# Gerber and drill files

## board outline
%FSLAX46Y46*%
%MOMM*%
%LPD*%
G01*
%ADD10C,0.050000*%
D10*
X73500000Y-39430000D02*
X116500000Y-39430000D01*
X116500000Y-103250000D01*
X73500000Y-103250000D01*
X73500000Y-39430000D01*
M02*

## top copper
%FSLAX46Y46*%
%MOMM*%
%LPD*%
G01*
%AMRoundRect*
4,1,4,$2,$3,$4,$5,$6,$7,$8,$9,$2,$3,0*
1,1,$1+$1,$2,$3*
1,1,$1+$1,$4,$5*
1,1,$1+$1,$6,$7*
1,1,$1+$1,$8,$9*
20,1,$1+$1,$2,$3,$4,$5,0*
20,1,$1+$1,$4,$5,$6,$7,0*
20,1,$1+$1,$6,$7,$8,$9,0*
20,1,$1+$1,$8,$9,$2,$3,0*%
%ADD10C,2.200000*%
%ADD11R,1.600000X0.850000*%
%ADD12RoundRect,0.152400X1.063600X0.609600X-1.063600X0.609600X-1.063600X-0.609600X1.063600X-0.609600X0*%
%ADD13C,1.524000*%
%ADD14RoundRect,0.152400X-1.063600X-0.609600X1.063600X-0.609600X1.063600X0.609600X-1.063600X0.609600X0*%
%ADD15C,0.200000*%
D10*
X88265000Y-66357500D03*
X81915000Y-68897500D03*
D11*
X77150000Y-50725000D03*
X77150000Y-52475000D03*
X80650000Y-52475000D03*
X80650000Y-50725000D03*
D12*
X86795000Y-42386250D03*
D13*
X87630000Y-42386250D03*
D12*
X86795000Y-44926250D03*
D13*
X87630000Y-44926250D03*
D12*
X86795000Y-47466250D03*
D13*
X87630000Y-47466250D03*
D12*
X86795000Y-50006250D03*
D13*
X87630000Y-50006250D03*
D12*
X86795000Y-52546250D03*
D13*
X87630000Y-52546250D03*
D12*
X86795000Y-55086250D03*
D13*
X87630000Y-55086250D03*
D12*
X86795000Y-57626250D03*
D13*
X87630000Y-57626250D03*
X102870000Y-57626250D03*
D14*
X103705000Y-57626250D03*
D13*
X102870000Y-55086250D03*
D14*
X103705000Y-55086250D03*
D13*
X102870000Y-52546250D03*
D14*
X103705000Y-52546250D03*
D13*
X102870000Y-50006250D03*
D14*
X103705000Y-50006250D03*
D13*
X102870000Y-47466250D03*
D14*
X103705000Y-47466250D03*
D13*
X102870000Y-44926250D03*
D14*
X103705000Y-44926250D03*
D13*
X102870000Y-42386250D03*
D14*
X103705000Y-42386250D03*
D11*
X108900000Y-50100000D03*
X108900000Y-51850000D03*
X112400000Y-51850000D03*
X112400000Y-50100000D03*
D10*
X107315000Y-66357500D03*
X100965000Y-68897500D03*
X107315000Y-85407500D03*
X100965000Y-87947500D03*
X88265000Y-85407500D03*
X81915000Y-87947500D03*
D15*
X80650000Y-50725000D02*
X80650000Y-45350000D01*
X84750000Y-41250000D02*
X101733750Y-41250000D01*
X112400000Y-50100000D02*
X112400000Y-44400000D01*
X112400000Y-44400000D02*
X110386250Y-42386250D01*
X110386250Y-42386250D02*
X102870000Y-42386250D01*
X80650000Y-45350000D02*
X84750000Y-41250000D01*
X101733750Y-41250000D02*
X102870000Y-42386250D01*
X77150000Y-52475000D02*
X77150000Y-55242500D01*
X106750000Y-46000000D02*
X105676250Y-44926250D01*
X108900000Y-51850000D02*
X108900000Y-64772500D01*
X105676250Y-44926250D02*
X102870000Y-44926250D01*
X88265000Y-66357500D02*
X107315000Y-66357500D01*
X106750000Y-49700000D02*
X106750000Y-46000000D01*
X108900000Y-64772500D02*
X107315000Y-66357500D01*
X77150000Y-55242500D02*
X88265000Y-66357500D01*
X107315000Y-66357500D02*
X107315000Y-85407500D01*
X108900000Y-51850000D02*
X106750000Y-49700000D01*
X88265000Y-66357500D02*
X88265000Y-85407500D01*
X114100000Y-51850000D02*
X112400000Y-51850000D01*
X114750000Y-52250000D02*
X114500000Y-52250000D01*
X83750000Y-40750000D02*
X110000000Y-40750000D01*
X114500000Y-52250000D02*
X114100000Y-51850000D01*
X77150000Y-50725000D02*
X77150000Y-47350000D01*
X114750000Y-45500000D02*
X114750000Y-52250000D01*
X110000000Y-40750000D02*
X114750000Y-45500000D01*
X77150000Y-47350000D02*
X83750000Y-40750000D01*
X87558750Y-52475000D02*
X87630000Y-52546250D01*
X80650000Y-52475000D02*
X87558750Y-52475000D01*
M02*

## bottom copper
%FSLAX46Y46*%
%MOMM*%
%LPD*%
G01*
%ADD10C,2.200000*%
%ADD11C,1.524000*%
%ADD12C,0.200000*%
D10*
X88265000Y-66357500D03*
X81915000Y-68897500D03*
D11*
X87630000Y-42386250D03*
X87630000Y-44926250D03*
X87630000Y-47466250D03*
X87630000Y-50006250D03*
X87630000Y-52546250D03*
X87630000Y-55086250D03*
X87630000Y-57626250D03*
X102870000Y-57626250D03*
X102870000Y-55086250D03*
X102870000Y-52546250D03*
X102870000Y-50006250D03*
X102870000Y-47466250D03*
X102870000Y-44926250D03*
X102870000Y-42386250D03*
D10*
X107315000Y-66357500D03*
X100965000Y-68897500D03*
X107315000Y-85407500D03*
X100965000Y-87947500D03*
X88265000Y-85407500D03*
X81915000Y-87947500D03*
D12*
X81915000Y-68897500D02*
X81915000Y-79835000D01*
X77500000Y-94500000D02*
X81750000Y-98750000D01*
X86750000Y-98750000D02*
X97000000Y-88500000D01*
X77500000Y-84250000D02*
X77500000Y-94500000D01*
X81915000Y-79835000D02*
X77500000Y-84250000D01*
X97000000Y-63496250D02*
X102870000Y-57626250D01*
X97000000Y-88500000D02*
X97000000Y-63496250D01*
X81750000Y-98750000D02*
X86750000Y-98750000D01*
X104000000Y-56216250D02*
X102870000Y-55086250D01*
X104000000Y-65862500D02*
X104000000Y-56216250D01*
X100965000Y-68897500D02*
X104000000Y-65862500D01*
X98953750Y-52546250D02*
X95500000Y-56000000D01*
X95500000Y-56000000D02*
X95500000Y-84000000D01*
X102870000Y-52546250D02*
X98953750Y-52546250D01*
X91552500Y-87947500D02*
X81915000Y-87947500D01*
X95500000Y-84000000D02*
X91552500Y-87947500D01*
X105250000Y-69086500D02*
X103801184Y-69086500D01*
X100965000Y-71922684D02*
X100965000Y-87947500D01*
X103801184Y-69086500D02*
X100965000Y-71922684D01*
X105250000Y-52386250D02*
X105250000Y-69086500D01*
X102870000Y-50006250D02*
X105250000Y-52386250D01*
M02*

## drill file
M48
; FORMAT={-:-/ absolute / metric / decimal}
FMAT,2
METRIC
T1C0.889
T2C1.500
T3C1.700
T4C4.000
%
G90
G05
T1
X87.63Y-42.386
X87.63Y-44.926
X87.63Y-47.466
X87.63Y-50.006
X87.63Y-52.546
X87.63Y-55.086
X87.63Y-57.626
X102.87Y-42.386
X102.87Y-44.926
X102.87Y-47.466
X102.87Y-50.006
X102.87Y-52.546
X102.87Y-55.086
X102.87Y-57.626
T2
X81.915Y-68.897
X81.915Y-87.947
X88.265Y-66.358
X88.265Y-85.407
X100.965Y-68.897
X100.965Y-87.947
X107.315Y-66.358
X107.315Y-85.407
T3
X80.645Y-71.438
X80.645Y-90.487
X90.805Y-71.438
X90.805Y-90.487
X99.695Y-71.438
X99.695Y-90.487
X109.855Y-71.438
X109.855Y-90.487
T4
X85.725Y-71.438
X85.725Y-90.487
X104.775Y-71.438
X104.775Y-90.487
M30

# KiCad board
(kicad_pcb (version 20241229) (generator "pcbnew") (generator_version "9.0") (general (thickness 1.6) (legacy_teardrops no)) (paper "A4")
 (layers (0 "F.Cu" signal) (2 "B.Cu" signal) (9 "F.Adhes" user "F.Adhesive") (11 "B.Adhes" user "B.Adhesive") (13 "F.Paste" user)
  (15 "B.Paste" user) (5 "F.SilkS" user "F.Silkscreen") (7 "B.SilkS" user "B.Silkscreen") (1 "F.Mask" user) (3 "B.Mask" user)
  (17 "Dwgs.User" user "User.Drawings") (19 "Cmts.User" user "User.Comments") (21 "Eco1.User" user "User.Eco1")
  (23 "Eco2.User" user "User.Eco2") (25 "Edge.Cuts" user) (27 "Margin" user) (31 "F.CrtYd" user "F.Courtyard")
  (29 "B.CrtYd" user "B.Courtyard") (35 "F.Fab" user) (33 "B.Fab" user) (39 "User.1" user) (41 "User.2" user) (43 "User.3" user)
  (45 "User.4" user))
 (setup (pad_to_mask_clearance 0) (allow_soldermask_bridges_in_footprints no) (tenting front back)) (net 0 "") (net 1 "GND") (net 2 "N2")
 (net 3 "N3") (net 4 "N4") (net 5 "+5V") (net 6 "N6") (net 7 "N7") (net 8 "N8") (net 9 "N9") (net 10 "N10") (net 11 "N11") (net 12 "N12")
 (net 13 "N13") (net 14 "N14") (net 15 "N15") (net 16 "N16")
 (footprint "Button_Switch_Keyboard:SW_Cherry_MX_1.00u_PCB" (layer "F.Cu") (at 88.265 66.3575)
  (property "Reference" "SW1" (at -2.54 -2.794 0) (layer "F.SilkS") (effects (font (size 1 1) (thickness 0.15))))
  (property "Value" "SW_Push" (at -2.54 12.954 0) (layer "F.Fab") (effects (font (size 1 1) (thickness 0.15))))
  (pad "" np_thru_hole circle (at -7.62 5.08) (size 1.7 1.7) (drill 1.7) (layers "*.Cu" "*.Mask"))
  (pad "" np_thru_hole circle (at -2.54 5.08) (size 4 4) (drill 4) (layers "*.Cu" "*.Mask"))
  (pad "" np_thru_hole circle (at 2.54 5.08) (size 1.7 1.7) (drill 1.7) (layers "*.Cu" "*.Mask"))
  (pad "1" thru_hole circle (at 0 0) (size 2.2 2.2) (drill 1.5) (layers "*.Cu" "*.Mask") (remove_unused_layers no) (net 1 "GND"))
  (pad "2" thru_hole circle (at -6.35 2.54) (size 2.2 2.2) (drill 1.5) (layers "*.Cu" "*.Mask") (remove_unused_layers no) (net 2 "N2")))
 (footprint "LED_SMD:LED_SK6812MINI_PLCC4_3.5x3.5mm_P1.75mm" (layer "F.Cu") (at 78.9 51.6)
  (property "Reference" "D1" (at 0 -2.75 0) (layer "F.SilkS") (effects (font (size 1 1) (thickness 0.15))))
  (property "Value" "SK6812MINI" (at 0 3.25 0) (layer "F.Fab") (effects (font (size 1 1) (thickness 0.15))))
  (pad "1" smd rect (at -1.75 -0.875) (size 1.6 0.85) (layers "F.Cu" "F.Mask" "F.Paste") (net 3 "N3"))
  (pad "2" smd rect (at -1.75 0.875) (size 1.6 0.85) (layers "F.Cu" "F.Mask" "F.Paste") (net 1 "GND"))
  (pad "3" smd rect (at 1.75 0.875) (size 1.6 0.85) (layers "F.Cu" "F.Mask" "F.Paste") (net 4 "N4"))
  (pad "4" smd rect (at 1.75 -0.875) (size 1.6 0.85) (layers "F.Cu" "F.Mask" "F.Paste") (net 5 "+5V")))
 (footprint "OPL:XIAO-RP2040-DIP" (layer "F.Cu") (at 95.25 50.00625)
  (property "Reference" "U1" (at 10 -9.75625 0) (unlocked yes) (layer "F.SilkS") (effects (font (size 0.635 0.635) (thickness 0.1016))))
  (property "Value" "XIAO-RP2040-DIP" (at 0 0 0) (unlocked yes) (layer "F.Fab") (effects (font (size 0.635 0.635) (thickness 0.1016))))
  (pad "1" smd roundrect (at -8.455 -7.62 180) (size 2.432 1.524) (layers "F.Cu" "F.Mask") (roundrect_rratio 0.1) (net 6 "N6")
   (thermal_bridge_angle 45))
  (pad "1" thru_hole circle (at -7.62 -7.62 180) (size 1.524 1.524) (drill 0.889) (layers "*.Cu" "*.Mask") (remove_unused_layers no)
   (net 6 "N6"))
  (pad "2" smd roundrect (at -8.455 -5.08 180) (size 2.432 1.524) (layers "F.Cu" "F.Mask") (roundrect_rratio 0.1) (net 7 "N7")
   (thermal_bridge_angle 45))
  (pad "2" thru_hole circle (at -7.62 -5.08 180) (size 1.524 1.524) (drill 0.889) (layers "*.Cu" "*.Mask") (remove_unused_layers no)
   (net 7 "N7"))
  (pad "3" smd roundrect (at -8.455 -2.54 180) (size 2.432 1.524) (layers "F.Cu" "F.Mask") (roundrect_rratio 0.1) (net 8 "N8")
   (thermal_bridge_angle 45))
  (pad "3" thru_hole circle (at -7.62 -2.54 180) (size 1.524 1.524) (drill 0.889) (layers "*.Cu" "*.Mask") (remove_unused_layers no)
   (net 8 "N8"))
  (pad "4" smd roundrect (at -8.455 0 180) (size 2.432 1.524) (layers "F.Cu" "F.Mask") (roundrect_rratio 0.1) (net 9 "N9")
   (thermal_bridge_angle 45))
  (pad "4" thru_hole circle (at -7.62 0 180) (size 1.524 1.524) (drill 0.889) (layers "*.Cu" "*.Mask") (remove_unused_layers no)
   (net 9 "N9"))
  (pad "5" smd roundrect (at -8.455 2.54 180) (size 2.432 1.524) (layers "F.Cu" "F.Mask") (roundrect_rratio 0.1) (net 4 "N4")
   (thermal_bridge_angle 45))
  (pad "5" thru_hole circle (at -7.62 2.54 180) (size 1.524 1.524) (drill 0.889) (layers "*.Cu" "*.Mask") (remove_unused_layers no)
   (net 4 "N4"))
  (pad "6" smd roundrect (at -8.455 5.08 180) (size 2.432 1.524) (layers "F.Cu" "F.Mask") (roundrect_rratio 0.1) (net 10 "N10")
   (thermal_bridge_angle 45))
  (pad "6" thru_hole circle (at -7.62 5.08 180) (size 1.524 1.524) (drill 0.889) (layers "*.Cu" "*.Mask") (remove_unused_layers no)
   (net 10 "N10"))
  (pad "7" smd roundrect (at -8.455 7.62 180) (size 2.432 1.524) (layers "F.Cu" "F.Mask") (roundrect_rratio 0.1) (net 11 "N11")
   (thermal_bridge_angle 45))
  (pad "7" thru_hole circle (at -7.62 7.62 180) (size 1.524 1.524) (drill 0.889) (layers "*.Cu" "*.Mask") (remove_unused_layers no)
   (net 11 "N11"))
  (pad "8" thru_hole circle (at 7.62 7.62) (size 1.524 1.524) (drill 0.889) (layers "*.Cu" "*.Mask") (remove_unused_layers no) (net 2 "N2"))
  (pad "8" smd roundrect (at 8.455 7.62) (size 2.432 1.524) (layers "F.Cu" "F.Mask") (roundrect_rratio 0.1) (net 2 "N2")
   (thermal_bridge_angle 45))
  (pad "9" thru_hole circle (at 7.62 5.08) (size 1.524 1.524) (drill 0.889) (layers "*.Cu" "*.Mask") (remove_unused_layers no)
   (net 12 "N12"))
  (pad "9" smd roundrect (at 8.455 5.08) (size 2.432 1.524) (layers "F.Cu" "F.Mask") (roundrect_rratio 0.1) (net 12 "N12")
   (thermal_bridge_angle 45))
  (pad "10" thru_hole circle (at 7.62 2.54) (size 1.524 1.524) (drill 0.889) (layers "*.Cu" "*.Mask") (remove_unused_layers no)
   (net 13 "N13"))
  (pad "10" smd roundrect (at 8.455 2.54) (size 2.432 1.524) (layers "F.Cu" "F.Mask") (roundrect_rratio 0.1) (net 13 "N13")
   (thermal_bridge_angle 45))
  (pad "11" thru_hole circle (at 7.62 0) (size 1.524 1.524) (drill 0.889) (layers "*.Cu" "*.Mask") (remove_unused_layers no) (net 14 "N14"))
  (pad "11" smd roundrect (at 8.455 0) (size 2.432 1.524) (layers "F.Cu" "F.Mask") (roundrect_rratio 0.1) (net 14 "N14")
   (thermal_bridge_angle 45))
  (pad "12" thru_hole circle (at 7.62 -2.54) (size 1.524 1.524) (drill 0.889) (layers "*.Cu" "*.Mask") (remove_unused_layers no)
   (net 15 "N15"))
  (pad "12" smd roundrect (at 8.455 -2.54) (size 2.432 1.524) (layers "F.Cu" "F.Mask") (roundrect_rratio 0.1) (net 15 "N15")
   (thermal_bridge_angle 45))
  (pad "13" thru_hole circle (at 7.62 -5.08) (size 1.524 1.524) (drill 0.889) (layers "*.Cu" "*.Mask") (remove_unused_layers no)
   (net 1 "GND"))
  (pad "13" smd roundrect (at 8.455 -5.08) (size 2.432 1.524) (layers "F.Cu" "F.Mask") (roundrect_rratio 0.1) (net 1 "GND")
   (thermal_bridge_angle 45))
  (pad "14" thru_hole circle (at 7.62 -7.62) (size 1.524 1.524) (drill 0.889) (layers "*.Cu" "*.Mask") (remove_unused_layers no)
   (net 5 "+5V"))
  (pad "14" smd roundrect (at 8.455 -7.62) (size 2.432 1.524) (layers "F.Cu" "F.Mask") (roundrect_rratio 0.1) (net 5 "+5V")
   (thermal_bridge_angle 45)))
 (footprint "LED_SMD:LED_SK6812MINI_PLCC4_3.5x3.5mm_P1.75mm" (layer "F.Cu") (at 110.65 50.975)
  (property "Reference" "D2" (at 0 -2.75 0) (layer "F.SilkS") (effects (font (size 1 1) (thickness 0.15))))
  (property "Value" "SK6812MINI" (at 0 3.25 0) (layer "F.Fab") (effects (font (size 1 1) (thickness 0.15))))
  (pad "1" smd rect (at -1.75 -0.875) (size 1.6 0.85) (layers "F.Cu" "F.Mask" "F.Paste") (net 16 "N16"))
  (pad "2" smd rect (at -1.75 0.875) (size 1.6 0.85) (layers "F.Cu" "F.Mask" "F.Paste") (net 1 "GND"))
  (pad "3" smd rect (at 1.75 0.875) (size 1.6 0.85) (layers "F.Cu" "F.Mask" "F.Paste") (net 3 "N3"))
  (pad "4" smd rect (at 1.75 -0.875) (size 1.6 0.85) (layers "F.Cu" "F.Mask" "F.Paste") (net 5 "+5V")))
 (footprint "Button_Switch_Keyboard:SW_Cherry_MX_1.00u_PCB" (layer "F.Cu") (at 107.315 66.3575)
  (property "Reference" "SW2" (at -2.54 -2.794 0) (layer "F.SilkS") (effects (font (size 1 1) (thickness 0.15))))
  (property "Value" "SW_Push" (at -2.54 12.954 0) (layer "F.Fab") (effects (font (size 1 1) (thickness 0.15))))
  (pad "" np_thru_hole circle (at -7.62 5.08) (size 1.7 1.7) (drill 1.7) (layers "*.Cu" "*.Mask"))
  (pad "" np_thru_hole circle (at -2.54 5.08) (size 4 4) (drill 4) (layers "*.Cu" "*.Mask"))
  (pad "" np_thru_hole circle (at 2.54 5.08) (size 1.7 1.7) (drill 1.7) (layers "*.Cu" "*.Mask"))
  (pad "1" thru_hole circle (at 0 0) (size 2.2 2.2) (drill 1.5) (layers "*.Cu" "*.Mask") (remove_unused_layers no) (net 1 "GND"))
  (pad "2" thru_hole circle (at -6.35 2.54) (size 2.2 2.2) (drill 1.5) (layers "*.Cu" "*.Mask") (remove_unused_layers no) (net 12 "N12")))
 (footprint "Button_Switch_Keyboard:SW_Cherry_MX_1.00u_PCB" (layer "F.Cu") (at 107.315 85.4075)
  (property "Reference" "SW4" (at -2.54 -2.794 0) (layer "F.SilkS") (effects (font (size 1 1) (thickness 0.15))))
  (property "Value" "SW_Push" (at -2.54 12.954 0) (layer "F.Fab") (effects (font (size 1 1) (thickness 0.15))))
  (pad "" np_thru_hole circle (at -7.62 5.08) (size 1.7 1.7) (drill 1.7) (layers "*.Cu" "*.Mask"))
  (pad "" np_thru_hole circle (at -2.54 5.08) (size 4 4) (drill 4) (layers "*.Cu" "*.Mask"))
  (pad "" np_thru_hole circle (at 2.54 5.08) (size 1.7 1.7) (drill 1.7) (layers "*.Cu" "*.Mask"))
  (pad "1" thru_hole circle (at 0 0) (size 2.2 2.2) (drill 1.5) (layers "*.Cu" "*.Mask") (remove_unused_layers no) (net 1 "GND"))
  (pad "2" thru_hole circle (at -6.35 2.54) (size 2.2 2.2) (drill 1.5) (layers "*.Cu" "*.Mask") (remove_unused_layers no) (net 14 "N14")))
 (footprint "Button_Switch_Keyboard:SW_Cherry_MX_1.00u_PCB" (layer "F.Cu") (at 88.265 85.4075)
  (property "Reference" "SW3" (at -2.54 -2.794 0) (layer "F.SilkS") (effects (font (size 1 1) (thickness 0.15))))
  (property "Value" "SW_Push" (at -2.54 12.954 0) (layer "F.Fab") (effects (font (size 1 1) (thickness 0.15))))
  (pad "" np_thru_hole circle (at -7.62 5.08) (size 1.7 1.7) (drill 1.7) (layers "*.Cu" "*.Mask"))
  (pad "" np_thru_hole circle (at -2.54 5.08) (size 4 4) (drill 4) (layers "*.Cu" "*.Mask"))
  (pad "" np_thru_hole circle (at 2.54 5.08) (size 1.7 1.7) (drill 1.7) (layers "*.Cu" "*.Mask"))
  (pad "1" thru_hole circle (at 0 0) (size 2.2 2.2) (drill 1.5) (layers "*.Cu" "*.Mask") (remove_unused_layers no) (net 1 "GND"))
  (pad "2" thru_hole circle (at -6.35 2.54) (size 2.2 2.2) (drill 1.5) (layers "*.Cu" "*.Mask") (remove_unused_layers no) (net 13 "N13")))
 (gr_rect (start 73.5 39.43) (end 116.5 103.25) (stroke (width 0.05) (type default)) (fill no) (layer "Edge.Cuts"))
 (segment (start 80.65 50.725) (end 80.65 45.35) (width 0.2) (layer "F.Cu") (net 5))
 (segment (start 84.75 41.25) (end 101.73375 41.25) (width 0.2) (layer "F.Cu") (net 5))
 (segment (start 112.4 50.1) (end 112.4 44.4) (width 0.2) (layer "F.Cu") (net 5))
 (segment (start 112.4 44.4) (end 110.38625 42.38625) (width 0.2) (layer "F.Cu") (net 5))
 (segment (start 110.38625 42.38625) (end 102.87 42.38625) (width 0.2) (layer "F.Cu") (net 5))
 (segment (start 80.65 45.35) (end 84.75 41.25) (width 0.2) (layer "F.Cu") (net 5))
 (segment (start 101.73375 41.25) (end 102.87 42.38625) (width 0.2) (layer "F.Cu") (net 5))
 (segment (start 77.15 52.475) (end 77.15 55.2425) (width 0.2) (layer "F.Cu") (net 1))
 (segment (start 106.75 46) (end 105.67625 44.92625) (width 0.2) (layer "F.Cu") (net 1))
 (segment (start 108.9 51.85) (end 108.9 64.7725) (width 0.2) (layer "F.Cu") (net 1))
 (segment (start 105.67625 44.92625) (end 102.87 44.92625) (width 0.2) (layer "F.Cu") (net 1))
 (segment (start 88.265 66.3575) (end 107.315 66.3575) (width 0.2) (layer "F.Cu") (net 1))
 (segment (start 106.75 49.7) (end 106.75 46) (width 0.2) (layer "F.Cu") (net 1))
 (segment (start 108.9 64.7725) (end 107.315 66.3575) (width 0.2) (layer "F.Cu") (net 1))
 (segment (start 77.15 55.2425) (end 88.265 66.3575) (width 0.2) (layer "F.Cu") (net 1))
 (segment (start 107.315 66.3575) (end 107.315 85.4075) (width 0.2) (layer "F.Cu") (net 1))
 (segment (start 108.9 51.85) (end 106.75 49.7) (width 0.2) (layer "F.Cu") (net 1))
 (segment (start 88.265 66.3575) (end 88.265 85.4075) (width 0.2) (layer "F.Cu") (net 1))
 (segment (start 114.1 51.85) (end 112.4 51.85) (width 0.2) (layer "F.Cu") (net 3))
 (segment (start 114.75 52.25) (end 114.5 52.25) (width 0.2) (layer "F.Cu") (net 3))
 (segment (start 83.75 40.75) (end 110 40.75) (width 0.2) (layer "F.Cu") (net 3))
 (segment (start 114.5 52.25) (end 114.1 51.85) (width 0.2) (layer "F.Cu") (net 3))
 (segment (start 77.15 50.725) (end 77.15 47.35) (width 0.2) (layer "F.Cu") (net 3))
 (segment (start 114.75 45.5) (end 114.75 52.25) (width 0.2) (layer "F.Cu") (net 3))
 (segment (start 110 40.75) (end 114.75 45.5) (width 0.2) (layer "F.Cu") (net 3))
 (segment (start 77.15 47.35) (end 83.75 40.75) (width 0.2) (layer "F.Cu") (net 3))
 (segment (start 87.55875 52.475) (end 87.63 52.54625) (width 0.2) (layer "F.Cu") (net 4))
 (segment (start 80.65 52.475) (end 87.55875 52.475) (width 0.2) (layer "F.Cu") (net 4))
 (segment (start 81.915 68.8975) (end 81.915 79.835) (width 0.2) (layer "B.Cu") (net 2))
 (segment (start 77.5 94.5) (end 81.75 98.75) (width 0.2) (layer "B.Cu") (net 2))
 (segment (start 86.75 98.75) (end 97 88.5) (width 0.2) (layer "B.Cu") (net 2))
 (segment (start 77.5 84.25) (end 77.5 94.5) (width 0.2) (layer "B.Cu") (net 2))
 (segment (start 81.915 79.835) (end 77.5 84.25) (width 0.2) (layer "B.Cu") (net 2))
 (segment (start 97 63.49625) (end 102.87 57.62625) (width 0.2) (layer "B.Cu") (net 2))
 (segment (start 97 88.5) (end 97 63.49625) (width 0.2) (layer "B.Cu") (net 2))
 (segment (start 81.75 98.75) (end 86.75 98.75) (width 0.2) (layer "B.Cu") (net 2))
 (segment (start 104 56.21625) (end 102.87 55.08625) (width 0.2) (layer "B.Cu") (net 12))
 (segment (start 104 65.8625) (end 104 56.21625) (width 0.2) (layer "B.Cu") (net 12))
 (segment (start 100.965 68.8975) (end 104 65.8625) (width 0.2) (layer "B.Cu") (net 12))
 (segment (start 98.95375 52.54625) (end 95.5 56) (width 0.2) (layer "B.Cu") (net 13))
 (segment (start 95.5 56) (end 95.5 84) (width 0.2) (layer "B.Cu") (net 13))
 (segment (start 102.87 52.54625) (end 98.95375 52.54625) (width 0.2) (layer "B.Cu") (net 13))
 (segment (start 91.5525 87.9475) (end 81.915 87.9475) (width 0.2) (layer "B.Cu") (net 13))
 (segment (start 95.5 84) (end 91.5525 87.9475) (width 0.2) (layer "B.Cu") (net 13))
 (segment (start 105.25 69.0865) (end 103.801184 69.0865) (width 0.2) (layer "B.Cu") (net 14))
 (segment (start 100.965 71.922684) (end 100.965 87.9475) (width 0.2) (layer "B.Cu") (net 14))
 (segment (start 103.801184 69.0865) (end 100.965 71.922684) (width 0.2) (layer "B.Cu") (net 14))
 (segment (start 105.25 52.38625) (end 105.25 69.0865) (width 0.2) (layer "B.Cu") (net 14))
 (segment (start 102.87 50.00625) (end 105.25 52.38625) (width 0.2) (layer "B.Cu") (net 14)))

